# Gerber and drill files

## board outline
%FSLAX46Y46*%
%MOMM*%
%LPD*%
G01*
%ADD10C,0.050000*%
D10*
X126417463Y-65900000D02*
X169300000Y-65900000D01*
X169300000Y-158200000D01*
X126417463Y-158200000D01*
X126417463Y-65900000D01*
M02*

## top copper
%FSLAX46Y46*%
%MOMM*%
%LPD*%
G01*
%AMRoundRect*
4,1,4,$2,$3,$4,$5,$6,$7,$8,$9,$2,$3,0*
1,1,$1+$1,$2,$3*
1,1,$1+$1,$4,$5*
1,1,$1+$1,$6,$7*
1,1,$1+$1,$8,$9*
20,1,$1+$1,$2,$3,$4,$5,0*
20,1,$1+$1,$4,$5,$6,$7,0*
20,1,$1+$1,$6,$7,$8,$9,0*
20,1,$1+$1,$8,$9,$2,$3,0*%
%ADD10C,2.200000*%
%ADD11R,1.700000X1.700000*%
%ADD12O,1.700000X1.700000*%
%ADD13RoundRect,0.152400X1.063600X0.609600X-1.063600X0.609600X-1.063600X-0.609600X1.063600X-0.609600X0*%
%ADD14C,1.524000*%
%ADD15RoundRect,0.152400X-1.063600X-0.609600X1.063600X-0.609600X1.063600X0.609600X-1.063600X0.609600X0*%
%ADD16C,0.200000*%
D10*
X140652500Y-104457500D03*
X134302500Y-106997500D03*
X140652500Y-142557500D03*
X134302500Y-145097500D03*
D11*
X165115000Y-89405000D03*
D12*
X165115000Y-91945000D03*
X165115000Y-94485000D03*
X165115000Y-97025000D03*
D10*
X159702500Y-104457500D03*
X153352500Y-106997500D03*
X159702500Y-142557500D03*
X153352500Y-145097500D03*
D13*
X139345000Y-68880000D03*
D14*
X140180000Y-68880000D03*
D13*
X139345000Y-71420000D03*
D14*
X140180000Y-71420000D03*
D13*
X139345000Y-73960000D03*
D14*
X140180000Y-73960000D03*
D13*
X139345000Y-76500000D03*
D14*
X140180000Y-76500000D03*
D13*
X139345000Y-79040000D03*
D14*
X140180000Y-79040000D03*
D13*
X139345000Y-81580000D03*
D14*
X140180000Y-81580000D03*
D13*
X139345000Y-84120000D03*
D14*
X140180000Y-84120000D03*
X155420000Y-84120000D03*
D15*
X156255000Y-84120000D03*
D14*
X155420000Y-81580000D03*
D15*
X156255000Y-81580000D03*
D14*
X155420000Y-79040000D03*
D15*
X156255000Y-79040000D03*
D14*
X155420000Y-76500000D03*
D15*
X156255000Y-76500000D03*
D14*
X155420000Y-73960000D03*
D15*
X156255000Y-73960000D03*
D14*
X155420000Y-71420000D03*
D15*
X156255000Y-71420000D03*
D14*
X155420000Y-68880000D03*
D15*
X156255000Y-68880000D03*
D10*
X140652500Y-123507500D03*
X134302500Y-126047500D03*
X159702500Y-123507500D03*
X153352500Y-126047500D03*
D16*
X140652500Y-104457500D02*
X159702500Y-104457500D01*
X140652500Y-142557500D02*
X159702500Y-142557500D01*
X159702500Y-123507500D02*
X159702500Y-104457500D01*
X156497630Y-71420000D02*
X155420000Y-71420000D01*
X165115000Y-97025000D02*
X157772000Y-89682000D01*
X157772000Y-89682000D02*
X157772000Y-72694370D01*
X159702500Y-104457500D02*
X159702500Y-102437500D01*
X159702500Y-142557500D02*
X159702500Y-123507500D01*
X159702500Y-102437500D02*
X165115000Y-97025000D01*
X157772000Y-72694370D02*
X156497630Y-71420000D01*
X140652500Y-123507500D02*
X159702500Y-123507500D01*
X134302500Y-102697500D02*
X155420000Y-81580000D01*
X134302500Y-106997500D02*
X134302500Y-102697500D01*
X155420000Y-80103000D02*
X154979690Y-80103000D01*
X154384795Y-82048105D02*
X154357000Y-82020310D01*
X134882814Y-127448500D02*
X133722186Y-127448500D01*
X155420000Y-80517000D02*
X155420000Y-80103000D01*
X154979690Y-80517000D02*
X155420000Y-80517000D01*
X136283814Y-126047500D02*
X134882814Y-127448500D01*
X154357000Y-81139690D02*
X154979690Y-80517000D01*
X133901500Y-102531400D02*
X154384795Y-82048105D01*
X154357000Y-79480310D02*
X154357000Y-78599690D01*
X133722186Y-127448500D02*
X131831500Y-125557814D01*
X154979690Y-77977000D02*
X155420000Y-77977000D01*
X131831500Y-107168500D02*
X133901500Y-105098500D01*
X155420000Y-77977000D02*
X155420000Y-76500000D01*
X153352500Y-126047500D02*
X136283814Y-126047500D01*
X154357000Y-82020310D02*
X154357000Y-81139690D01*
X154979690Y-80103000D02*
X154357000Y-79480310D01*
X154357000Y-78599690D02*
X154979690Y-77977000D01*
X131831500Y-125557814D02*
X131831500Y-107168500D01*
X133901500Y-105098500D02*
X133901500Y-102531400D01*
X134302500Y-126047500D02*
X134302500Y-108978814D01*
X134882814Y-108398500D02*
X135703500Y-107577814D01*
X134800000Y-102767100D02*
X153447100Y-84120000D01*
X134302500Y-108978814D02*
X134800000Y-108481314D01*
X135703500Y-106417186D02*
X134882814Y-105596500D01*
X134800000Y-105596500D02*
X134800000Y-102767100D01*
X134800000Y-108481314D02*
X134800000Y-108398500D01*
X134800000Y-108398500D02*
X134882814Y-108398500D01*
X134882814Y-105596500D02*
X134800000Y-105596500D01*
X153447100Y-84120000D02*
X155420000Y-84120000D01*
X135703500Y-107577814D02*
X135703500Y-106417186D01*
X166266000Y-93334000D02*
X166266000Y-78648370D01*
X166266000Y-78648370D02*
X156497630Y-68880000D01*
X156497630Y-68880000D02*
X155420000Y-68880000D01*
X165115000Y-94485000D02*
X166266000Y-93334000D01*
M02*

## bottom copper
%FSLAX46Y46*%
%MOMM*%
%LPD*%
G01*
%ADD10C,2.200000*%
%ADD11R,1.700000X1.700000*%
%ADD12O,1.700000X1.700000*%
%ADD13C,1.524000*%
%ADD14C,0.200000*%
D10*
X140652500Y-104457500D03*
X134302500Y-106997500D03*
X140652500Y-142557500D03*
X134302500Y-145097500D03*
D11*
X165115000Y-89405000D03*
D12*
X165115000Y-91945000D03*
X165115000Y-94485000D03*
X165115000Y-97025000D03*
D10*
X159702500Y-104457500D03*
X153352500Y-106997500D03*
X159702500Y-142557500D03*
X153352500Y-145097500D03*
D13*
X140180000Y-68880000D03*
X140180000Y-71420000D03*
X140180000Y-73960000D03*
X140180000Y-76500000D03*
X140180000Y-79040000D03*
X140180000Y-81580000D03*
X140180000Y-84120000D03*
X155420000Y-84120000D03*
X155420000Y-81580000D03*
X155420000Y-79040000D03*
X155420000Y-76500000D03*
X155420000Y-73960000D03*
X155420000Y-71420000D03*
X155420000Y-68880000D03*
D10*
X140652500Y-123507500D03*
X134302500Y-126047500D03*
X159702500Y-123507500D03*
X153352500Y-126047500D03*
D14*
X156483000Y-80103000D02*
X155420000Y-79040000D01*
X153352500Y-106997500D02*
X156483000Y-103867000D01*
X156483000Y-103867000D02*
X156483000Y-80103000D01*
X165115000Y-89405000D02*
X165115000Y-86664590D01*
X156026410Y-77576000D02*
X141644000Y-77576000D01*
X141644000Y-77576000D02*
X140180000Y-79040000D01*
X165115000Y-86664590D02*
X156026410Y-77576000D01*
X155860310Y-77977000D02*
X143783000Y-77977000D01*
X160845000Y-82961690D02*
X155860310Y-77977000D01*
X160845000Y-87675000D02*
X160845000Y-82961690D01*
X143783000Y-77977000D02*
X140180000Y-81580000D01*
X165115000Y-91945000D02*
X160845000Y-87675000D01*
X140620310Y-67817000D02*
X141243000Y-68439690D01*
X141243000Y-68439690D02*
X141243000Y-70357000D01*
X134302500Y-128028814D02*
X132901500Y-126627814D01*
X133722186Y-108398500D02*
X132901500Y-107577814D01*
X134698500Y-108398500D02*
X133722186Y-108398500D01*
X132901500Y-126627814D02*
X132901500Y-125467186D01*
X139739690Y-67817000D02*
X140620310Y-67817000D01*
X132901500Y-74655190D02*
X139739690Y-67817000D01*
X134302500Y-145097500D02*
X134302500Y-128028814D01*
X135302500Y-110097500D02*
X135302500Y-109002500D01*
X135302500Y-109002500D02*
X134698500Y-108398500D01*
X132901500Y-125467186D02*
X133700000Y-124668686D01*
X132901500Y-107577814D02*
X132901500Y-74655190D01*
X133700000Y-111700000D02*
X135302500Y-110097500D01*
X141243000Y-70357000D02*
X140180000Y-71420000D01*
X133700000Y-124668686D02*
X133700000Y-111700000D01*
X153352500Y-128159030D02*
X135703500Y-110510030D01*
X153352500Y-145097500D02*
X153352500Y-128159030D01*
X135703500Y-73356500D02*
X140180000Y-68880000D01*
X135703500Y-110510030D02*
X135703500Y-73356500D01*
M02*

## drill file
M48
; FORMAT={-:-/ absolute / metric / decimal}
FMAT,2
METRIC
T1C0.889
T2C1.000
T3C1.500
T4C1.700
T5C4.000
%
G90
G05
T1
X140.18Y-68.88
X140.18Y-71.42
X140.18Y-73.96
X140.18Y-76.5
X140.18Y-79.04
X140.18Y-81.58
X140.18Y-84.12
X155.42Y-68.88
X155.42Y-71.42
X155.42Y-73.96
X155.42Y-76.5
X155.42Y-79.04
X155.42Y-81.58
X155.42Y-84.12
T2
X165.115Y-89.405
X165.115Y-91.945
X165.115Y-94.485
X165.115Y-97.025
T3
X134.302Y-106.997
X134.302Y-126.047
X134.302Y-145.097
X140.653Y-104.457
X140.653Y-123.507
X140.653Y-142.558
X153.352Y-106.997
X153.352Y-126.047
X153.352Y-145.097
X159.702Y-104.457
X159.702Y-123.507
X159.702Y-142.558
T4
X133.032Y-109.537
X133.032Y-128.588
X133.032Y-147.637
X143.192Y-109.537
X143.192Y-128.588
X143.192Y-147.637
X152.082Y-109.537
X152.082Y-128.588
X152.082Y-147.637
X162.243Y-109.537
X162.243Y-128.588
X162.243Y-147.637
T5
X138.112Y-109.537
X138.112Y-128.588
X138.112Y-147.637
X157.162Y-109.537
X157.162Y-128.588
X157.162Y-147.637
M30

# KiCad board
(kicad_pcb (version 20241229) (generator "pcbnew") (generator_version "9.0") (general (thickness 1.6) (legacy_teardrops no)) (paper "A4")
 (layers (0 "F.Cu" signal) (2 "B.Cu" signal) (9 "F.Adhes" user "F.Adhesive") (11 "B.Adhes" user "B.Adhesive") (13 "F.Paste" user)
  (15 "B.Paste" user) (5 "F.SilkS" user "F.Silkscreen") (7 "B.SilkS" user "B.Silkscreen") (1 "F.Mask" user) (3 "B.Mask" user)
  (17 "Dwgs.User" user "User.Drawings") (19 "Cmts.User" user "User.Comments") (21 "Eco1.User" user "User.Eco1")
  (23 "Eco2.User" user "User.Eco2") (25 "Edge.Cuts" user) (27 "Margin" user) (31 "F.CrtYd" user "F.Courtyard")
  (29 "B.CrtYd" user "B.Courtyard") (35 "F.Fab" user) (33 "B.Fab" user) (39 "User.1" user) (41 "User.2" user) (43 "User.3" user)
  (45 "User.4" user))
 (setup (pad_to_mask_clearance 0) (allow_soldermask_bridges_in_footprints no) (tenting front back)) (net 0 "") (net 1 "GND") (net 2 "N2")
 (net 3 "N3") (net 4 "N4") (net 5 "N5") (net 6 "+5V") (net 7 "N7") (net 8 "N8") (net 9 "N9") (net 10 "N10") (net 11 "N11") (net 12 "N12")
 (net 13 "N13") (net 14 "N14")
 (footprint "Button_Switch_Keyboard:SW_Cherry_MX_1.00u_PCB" (layer "F.Cu") (at 140.6525 104.4575)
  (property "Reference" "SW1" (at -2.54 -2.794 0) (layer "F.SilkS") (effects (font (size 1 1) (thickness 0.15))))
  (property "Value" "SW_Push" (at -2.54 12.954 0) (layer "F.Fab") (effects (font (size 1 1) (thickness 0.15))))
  (pad "" np_thru_hole circle (at -7.62 5.08) (size 1.7 1.7) (drill 1.7) (layers "*.Cu" "*.Mask"))
  (pad "" np_thru_hole circle (at -2.54 5.08) (size 4 4) (drill 4) (layers "*.Cu" "*.Mask"))
  (pad "" np_thru_hole circle (at 2.54 5.08) (size 1.7 1.7) (drill 1.7) (layers "*.Cu" "*.Mask"))
  (pad "1" thru_hole circle (at 0 0) (size 2.2 2.2) (drill 1.5) (layers "*.Cu" "*.Mask") (remove_unused_layers no) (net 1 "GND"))
  (pad "2" thru_hole circle (at -6.35 2.54) (size 2.2 2.2) (drill 1.5) (layers "*.Cu" "*.Mask") (remove_unused_layers no) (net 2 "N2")))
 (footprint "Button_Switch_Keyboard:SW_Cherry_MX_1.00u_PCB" (layer "F.Cu") (at 140.6525 142.5575)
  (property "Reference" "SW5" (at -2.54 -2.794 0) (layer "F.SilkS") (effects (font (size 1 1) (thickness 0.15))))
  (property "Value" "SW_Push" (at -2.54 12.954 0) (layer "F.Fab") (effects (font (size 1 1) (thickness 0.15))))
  (pad "" np_thru_hole circle (at -7.62 5.08) (size 1.7 1.7) (drill 1.7) (layers "*.Cu" "*.Mask"))
  (pad "" np_thru_hole circle (at -2.54 5.08) (size 4 4) (drill 4) (layers "*.Cu" "*.Mask"))
  (pad "" np_thru_hole circle (at 2.54 5.08) (size 1.7 1.7) (drill 1.7) (layers "*.Cu" "*.Mask"))
  (pad "1" thru_hole circle (at 0 0) (size 2.2 2.2) (drill 1.5) (layers "*.Cu" "*.Mask") (remove_unused_layers no) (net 1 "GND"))
  (pad "2" thru_hole circle (at -6.35 2.54) (size 2.2 2.2) (drill 1.5) (layers "*.Cu" "*.Mask") (remove_unused_layers no) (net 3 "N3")))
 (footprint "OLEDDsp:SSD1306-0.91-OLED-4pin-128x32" (layer "F.Cu") (at 128.615 87.215)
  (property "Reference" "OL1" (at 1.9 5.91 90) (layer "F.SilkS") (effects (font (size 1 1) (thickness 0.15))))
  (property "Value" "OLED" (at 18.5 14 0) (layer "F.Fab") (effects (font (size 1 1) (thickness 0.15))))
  (pad "1" thru_hole rect (at 36.5 2.19) (size 1.7 1.7) (drill 1) (layers "*.Cu" "*.Mask") (remove_unused_layers no) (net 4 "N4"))
  (pad "2" thru_hole oval (at 36.5 4.73) (size 1.7 1.7) (drill 1) (layers "*.Cu" "*.Mask") (remove_unused_layers no) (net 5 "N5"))
  (pad "3" thru_hole oval (at 36.5 7.27) (size 1.7 1.7) (drill 1) (layers "*.Cu" "*.Mask") (remove_unused_layers no) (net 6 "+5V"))
  (pad "4" thru_hole oval (at 36.5 9.81) (size 1.7 1.7) (drill 1) (layers "*.Cu" "*.Mask") (remove_unused_layers no) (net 1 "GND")))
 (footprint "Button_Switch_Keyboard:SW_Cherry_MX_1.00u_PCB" (layer "F.Cu") (at 159.7025 104.4575)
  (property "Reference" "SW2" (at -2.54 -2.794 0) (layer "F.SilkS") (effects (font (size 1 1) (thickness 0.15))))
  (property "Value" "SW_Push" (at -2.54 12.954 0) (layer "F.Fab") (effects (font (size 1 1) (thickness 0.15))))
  (pad "" np_thru_hole circle (at -7.62 5.08) (size 1.7 1.7) (drill 1.7) (layers "*.Cu" "*.Mask"))
  (pad "" np_thru_hole circle (at -2.54 5.08) (size 4 4) (drill 4) (layers "*.Cu" "*.Mask"))
  (pad "" np_thru_hole circle (at 2.54 5.08) (size 1.7 1.7) (drill 1.7) (layers "*.Cu" "*.Mask"))
  (pad "1" thru_hole circle (at 0 0) (size 2.2 2.2) (drill 1.5) (layers "*.Cu" "*.Mask") (remove_unused_layers no) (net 1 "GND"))
  (pad "2" thru_hole circle (at -6.35 2.54) (size 2.2 2.2) (drill 1.5) (layers "*.Cu" "*.Mask") (remove_unused_layers no) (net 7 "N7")))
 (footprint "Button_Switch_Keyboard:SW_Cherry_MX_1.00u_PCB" (layer "F.Cu") (at 159.7025 142.5575)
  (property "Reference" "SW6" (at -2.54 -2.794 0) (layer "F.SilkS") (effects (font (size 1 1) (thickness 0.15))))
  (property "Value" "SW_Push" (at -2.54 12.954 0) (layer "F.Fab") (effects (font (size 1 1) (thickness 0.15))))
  (pad "" np_thru_hole circle (at -7.62 5.08) (size 1.7 1.7) (drill 1.7) (layers "*.Cu" "*.Mask"))
  (pad "" np_thru_hole circle (at -2.54 5.08) (size 4 4) (drill 4) (layers "*.Cu" "*.Mask"))
  (pad "" np_thru_hole circle (at 2.54 5.08) (size 1.7 1.7) (drill 1.7) (layers "*.Cu" "*.Mask"))
  (pad "1" thru_hole circle (at 0 0) (size 2.2 2.2) (drill 1.5) (layers "*.Cu" "*.Mask") (remove_unused_layers no) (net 1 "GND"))
  (pad "2" thru_hole circle (at -6.35 2.54) (size 2.2 2.2) (drill 1.5) (layers "*.Cu" "*.Mask") (remove_unused_layers no) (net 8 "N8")))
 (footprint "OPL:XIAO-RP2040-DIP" (layer "F.Cu") (at 147.8 76.5)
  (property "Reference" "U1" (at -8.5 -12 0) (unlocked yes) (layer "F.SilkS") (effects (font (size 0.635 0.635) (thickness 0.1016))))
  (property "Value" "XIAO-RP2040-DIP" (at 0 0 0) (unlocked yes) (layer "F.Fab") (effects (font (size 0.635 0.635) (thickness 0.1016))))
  (pad "1" smd roundrect (at -8.455 -7.62 180) (size 2.432 1.524) (layers "F.Cu" "F.Mask") (roundrect_rratio 0.1) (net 8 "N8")
   (thermal_bridge_angle 45))
  (pad "1" thru_hole circle (at -7.62 -7.62 180) (size 1.524 1.524) (drill 0.889) (layers "*.Cu" "*.Mask") (remove_unused_layers no)
   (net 8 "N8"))
  (pad "2" smd roundrect (at -8.455 -5.08 180) (size 2.432 1.524) (layers "F.Cu" "F.Mask") (roundrect_rratio 0.1) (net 3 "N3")
   (thermal_bridge_angle 45))
  (pad "2" thru_hole circle (at -7.62 -5.08 180) (size 1.524 1.524) (drill 0.889) (layers "*.Cu" "*.Mask") (remove_unused_layers no)
   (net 3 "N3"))
  (pad "3" smd roundrect (at -8.455 -2.54 180) (size 2.432 1.524) (layers "F.Cu" "F.Mask") (roundrect_rratio 0.1) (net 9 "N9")
   (thermal_bridge_angle 45))
  (pad "3" thru_hole circle (at -7.62 -2.54 180) (size 1.524 1.524) (drill 0.889) (layers "*.Cu" "*.Mask") (remove_unused_layers no)
   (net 9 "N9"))
  (pad "4" smd roundrect (at -8.455 0 180) (size 2.432 1.524) (layers "F.Cu" "F.Mask") (roundrect_rratio 0.1) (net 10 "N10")
   (thermal_bridge_angle 45))
  (pad "4" thru_hole circle (at -7.62 0 180) (size 1.524 1.524) (drill 0.889) (layers "*.Cu" "*.Mask") (remove_unused_layers no)
   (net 10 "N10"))
  (pad "5" smd roundrect (at -8.455 2.54 180) (size 2.432 1.524) (layers "F.Cu" "F.Mask") (roundrect_rratio 0.1) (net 4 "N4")
   (thermal_bridge_angle 45))
  (pad "5" thru_hole circle (at -7.62 2.54 180) (size 1.524 1.524) (drill 0.889) (layers "*.Cu" "*.Mask") (remove_unused_layers no)
   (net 4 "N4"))
  (pad "6" smd roundrect (at -8.455 5.08 180) (size 2.432 1.524) (layers "F.Cu" "F.Mask") (roundrect_rratio 0.1) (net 5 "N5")
   (thermal_bridge_angle 45))
  (pad "6" thru_hole circle (at -7.62 5.08 180) (size 1.524 1.524) (drill 0.889) (layers "*.Cu" "*.Mask") (remove_unused_layers no)
   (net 5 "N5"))
  (pad "7" smd roundrect (at -8.455 7.62 180) (size 2.432 1.524) (layers "F.Cu" "F.Mask") (roundrect_rratio 0.1) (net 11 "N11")
   (thermal_bridge_angle 45))
  (pad "7" thru_hole circle (at -7.62 7.62 180) (size 1.524 1.524) (drill 0.889) (layers "*.Cu" "*.Mask") (remove_unused_layers no)
   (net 11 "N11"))
  (pad "8" thru_hole circle (at 7.62 7.62) (size 1.524 1.524) (drill 0.889) (layers "*.Cu" "*.Mask") (remove_unused_layers no)
   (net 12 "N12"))
  (pad "8" smd roundrect (at 8.455 7.62) (size 2.432 1.524) (layers "F.Cu" "F.Mask") (roundrect_rratio 0.1) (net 12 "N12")
   (thermal_bridge_angle 45))
  (pad "9" thru_hole circle (at 7.62 5.08) (size 1.524 1.524) (drill 0.889) (layers "*.Cu" "*.Mask") (remove_unused_layers no) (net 2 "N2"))
  (pad "9" smd roundrect (at 8.455 5.08) (size 2.432 1.524) (layers "F.Cu" "F.Mask") (roundrect_rratio 0.1) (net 2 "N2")
   (thermal_bridge_angle 45))
  (pad "10" thru_hole circle (at 7.62 2.54) (size 1.524 1.524) (drill 0.889) (layers "*.Cu" "*.Mask") (remove_unused_layers no) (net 7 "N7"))
  (pad "10" smd roundrect (at 8.455 2.54) (size 2.432 1.524) (layers "F.Cu" "F.Mask") (roundrect_rratio 0.1) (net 7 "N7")
   (thermal_bridge_angle 45))
  (pad "11" thru_hole circle (at 7.62 0) (size 1.524 1.524) (drill 0.889) (layers "*.Cu" "*.Mask") (remove_unused_layers no) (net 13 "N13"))
  (pad "11" smd roundrect (at 8.455 0) (size 2.432 1.524) (layers "F.Cu" "F.Mask") (roundrect_rratio 0.1) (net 13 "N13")
   (thermal_bridge_angle 45))
  (pad "12" thru_hole circle (at 7.62 -2.54) (size 1.524 1.524) (drill 0.889) (layers "*.Cu" "*.Mask") (remove_unused_layers no)
   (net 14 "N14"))
  (pad "12" smd roundrect (at 8.455 -2.54) (size 2.432 1.524) (layers "F.Cu" "F.Mask") (roundrect_rratio 0.1) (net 14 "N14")
   (thermal_bridge_angle 45))
  (pad "13" thru_hole circle (at 7.62 -5.08) (size 1.524 1.524) (drill 0.889) (layers "*.Cu" "*.Mask") (remove_unused_layers no)
   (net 1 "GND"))
  (pad "13" smd roundrect (at 8.455 -5.08) (size 2.432 1.524) (layers "F.Cu" "F.Mask") (roundrect_rratio 0.1) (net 1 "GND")
   (thermal_bridge_angle 45))
  (pad "14" thru_hole circle (at 7.62 -7.62) (size 1.524 1.524) (drill 0.889) (layers "*.Cu" "*.Mask") (remove_unused_layers no)
   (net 6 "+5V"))
  (pad "14" smd roundrect (at 8.455 -7.62) (size 2.432 1.524) (layers "F.Cu" "F.Mask") (roundrect_rratio 0.1) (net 6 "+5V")
   (thermal_bridge_angle 45)))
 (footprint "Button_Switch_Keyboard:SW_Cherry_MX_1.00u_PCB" (layer "F.Cu") (at 140.6525 123.5075)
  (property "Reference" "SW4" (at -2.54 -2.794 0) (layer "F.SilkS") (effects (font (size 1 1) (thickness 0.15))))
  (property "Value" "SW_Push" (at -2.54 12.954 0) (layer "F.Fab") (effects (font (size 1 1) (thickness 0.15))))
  (pad "" np_thru_hole circle (at -7.62 5.08) (size 1.7 1.7) (drill 1.7) (layers "*.Cu" "*.Mask"))
  (pad "" np_thru_hole circle (at -2.54 5.08) (size 4 4) (drill 4) (layers "*.Cu" "*.Mask"))
  (pad "" np_thru_hole circle (at 2.54 5.08) (size 1.7 1.7) (drill 1.7) (layers "*.Cu" "*.Mask"))
  (pad "1" thru_hole circle (at 0 0) (size 2.2 2.2) (drill 1.5) (layers "*.Cu" "*.Mask") (remove_unused_layers no) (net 1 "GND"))
  (pad "2" thru_hole circle (at -6.35 2.54) (size 2.2 2.2) (drill 1.5) (layers "*.Cu" "*.Mask") (remove_unused_layers no) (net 12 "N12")))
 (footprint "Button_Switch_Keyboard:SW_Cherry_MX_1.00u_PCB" (layer "F.Cu") (at 159.7025 123.5075)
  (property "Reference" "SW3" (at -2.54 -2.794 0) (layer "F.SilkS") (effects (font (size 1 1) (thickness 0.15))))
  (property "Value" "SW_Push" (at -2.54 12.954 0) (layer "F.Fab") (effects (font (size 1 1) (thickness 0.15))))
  (pad "" np_thru_hole circle (at -7.62 5.08) (size 1.7 1.7) (drill 1.7) (layers "*.Cu" "*.Mask"))
  (pad "" np_thru_hole circle (at -2.54 5.08) (size 4 4) (drill 4) (layers "*.Cu" "*.Mask"))
  (pad "" np_thru_hole circle (at 2.54 5.08) (size 1.7 1.7) (drill 1.7) (layers "*.Cu" "*.Mask"))
  (pad "1" thru_hole circle (at 0 0) (size 2.2 2.2) (drill 1.5) (layers "*.Cu" "*.Mask") (remove_unused_layers no) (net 1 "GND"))
  (pad "2" thru_hole circle (at -6.35 2.54) (size 2.2 2.2) (drill 1.5) (layers "*.Cu" "*.Mask") (remove_unused_layers no) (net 13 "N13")))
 (gr_rect (start 126.417463 65.9) (end 169.3 158.2) (stroke (width 0.05) (type default)) (fill no) (layer "Edge.Cuts"))
 (segment (start 140.6525 104.4575) (end 159.7025 104.4575) (width 0.2) (layer "F.Cu") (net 1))
 (segment (start 140.6525 142.5575) (end 159.7025 142.5575) (width 0.2) (layer "F.Cu") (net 1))
 (segment (start 159.7025 123.5075) (end 159.7025 104.4575) (width 0.2) (layer "F.Cu") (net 1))
 (segment (start 156.49763 71.42) (end 155.42 71.42) (width 0.2) (layer "F.Cu") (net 1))
 (segment (start 165.115 97.025) (end 157.772 89.682) (width 0.2) (layer "F.Cu") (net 1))
 (segment (start 157.772 89.682) (end 157.772 72.69437) (width 0.2) (layer "F.Cu") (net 1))
 (segment (start 159.7025 104.4575) (end 159.7025 102.4375) (width 0.2) (layer "F.Cu") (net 1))
 (segment (start 159.7025 142.5575) (end 159.7025 123.5075) (width 0.2) (layer "F.Cu") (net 1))
 (segment (start 159.7025 102.4375) (end 165.115 97.025) (width 0.2) (layer "F.Cu") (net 1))
 (segment (start 157.772 72.69437) (end 156.49763 71.42) (width 0.2) (layer "F.Cu") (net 1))
 (segment (start 140.6525 123.5075) (end 159.7025 123.5075) (width 0.2) (layer "F.Cu") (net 1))
 (segment (start 134.3025 102.6975) (end 155.42 81.58) (width 0.2) (layer "F.Cu") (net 2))
 (segment (start 134.3025 106.9975) (end 134.3025 102.6975) (width 0.2) (layer "F.Cu") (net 2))
 (segment (start 156.483 80.103) (end 155.42 79.04) (width 0.2) (layer "B.Cu") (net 7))
 (segment (start 153.3525 106.9975) (end 156.483 103.867) (width 0.2) (layer "B.Cu") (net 7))
 (segment (start 156.483 103.867) (end 156.483 80.103) (width 0.2) (layer "B.Cu") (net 7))
 (segment (start 155.42 80.103) (end 154.97969 80.103) (width 0.2) (layer "F.Cu") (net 13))
 (segment (start 154.384795 82.048105) (end 154.357 82.02031) (width 0.2) (layer "F.Cu") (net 13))
 (segment (start 134.882814 127.4485) (end 133.722186 127.4485) (width 0.2) (layer "F.Cu") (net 13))
 (segment (start 155.42 80.517) (end 155.42 80.103) (width 0.2) (layer "F.Cu") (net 13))
 (segment (start 154.97969 80.517) (end 155.42 80.517) (width 0.2) (layer "F.Cu") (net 13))
 (segment (start 136.283814 126.0475) (end 134.882814 127.4485) (width 0.2) (layer "F.Cu") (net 13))
 (segment (start 154.357 81.13969) (end 154.97969 80.517) (width 0.2) (layer "F.Cu") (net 13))
 (segment (start 133.9015 102.5314) (end 154.384795 82.048105) (width 0.2) (layer "F.Cu") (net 13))
 (segment (start 154.357 79.48031) (end 154.357 78.59969) (width 0.2) (layer "F.Cu") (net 13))
 (segment (start 133.722186 127.4485) (end 131.8315 125.557814) (width 0.2) (layer "F.Cu") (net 13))
 (segment (start 154.97969 77.977) (end 155.42 77.977) (width 0.2) (layer "F.Cu") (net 13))
 (segment (start 131.8315 107.1685) (end 133.9015 105.0985) (width 0.2) (layer "F.Cu") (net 13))
 (segment (start 155.42 77.977) (end 155.42 76.5) (width 0.2) (layer "F.Cu") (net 13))
 (segment (start 153.3525 126.0475) (end 136.283814 126.0475) (width 0.2) (layer "F.Cu") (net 13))
 (segment (start 154.357 82.02031) (end 154.357 81.13969) (width 0.2) (layer "F.Cu") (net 13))
 (segment (start 154.97969 80.103) (end 154.357 79.48031) (width 0.2) (layer "F.Cu") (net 13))
 (segment (start 154.357 78.59969) (end 154.97969 77.977) (width 0.2) (layer "F.Cu") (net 13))
 (segment (start 131.8315 125.557814) (end 131.8315 107.1685) (width 0.2) (layer "F.Cu") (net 13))
 (segment (start 133.9015 105.0985) (end 133.9015 102.5314) (width 0.2) (layer "F.Cu") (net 13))
 (segment (start 134.3025 126.0475) (end 134.3025 108.978814) (width 0.2) (layer "F.Cu") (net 12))
 (segment (start 134.882814 108.3985) (end 135.7035 107.577814) (width 0.2) (layer "F.Cu") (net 12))
 (segment (start 134.8 102.7671) (end 153.4471 84.12) (width 0.2) (layer "F.Cu") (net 12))
 (segment (start 134.3025 108.978814) (end 134.8 108.481314) (width 0.2) (layer "F.Cu") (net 12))
 (segment (start 135.7035 106.417186) (end 134.882814 105.5965) (width 0.2) (layer "F.Cu") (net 12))
 (segment (start 134.8 105.5965) (end 134.8 102.7671) (width 0.2) (layer "F.Cu") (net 12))
 (segment (start 134.8 108.481314) (end 134.8 108.3985) (width 0.2) (layer "F.Cu") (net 12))
 (segment (start 134.8 108.3985) (end 134.882814 108.3985) (width 0.2) (layer "F.Cu") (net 12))
 (segment (start 134.882814 105.5965) (end 134.8 105.5965) (width 0.2) (layer "F.Cu") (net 12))
 (segment (start 153.4471 84.12) (end 155.42 84.12) (width 0.2) (layer "F.Cu") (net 12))
 (segment (start 135.7035 107.577814) (end 135.7035 106.417186) (width 0.2) (layer "F.Cu") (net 12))
 (segment (start 165.115 89.405) (end 165.115 86.66459) (width 0.2) (layer "B.Cu") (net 4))
 (segment (start 156.02641 77.576) (end 141.644 77.576) (width 0.2) (layer "B.Cu") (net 4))
 (segment (start 141.644 77.576) (end 140.18 79.04) (width 0.2) (layer "B.Cu") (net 4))
 (segment (start 165.115 86.66459) (end 156.02641 77.576) (width 0.2) (layer "B.Cu") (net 4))
 (segment (start 155.86031 77.977) (end 143.783 77.977) (width 0.2) (layer "B.Cu") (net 5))
 (segment (start 160.845 82.96169) (end 155.86031 77.977) (width 0.2) (layer "B.Cu") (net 5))
 (segment (start 160.845 87.675) (end 160.845 82.96169) (width 0.2) (layer "B.Cu") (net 5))
 (segment (start 143.783 77.977) (end 140.18 81.58) (width 0.2) (layer "B.Cu") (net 5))
 (segment (start 165.115 91.945) (end 160.845 87.675) (width 0.2) (layer "B.Cu") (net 5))
 (segment (start 166.266 93.334) (end 166.266 78.64837) (width 0.2) (layer "F.Cu") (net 6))
 (segment (start 166.266 78.64837) (end 156.49763 68.88) (width 0.2) (layer "F.Cu") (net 6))
 (segment (start 156.49763 68.88) (end 155.42 68.88) (width 0.2) (layer "F.Cu") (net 6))
 (segment (start 165.115 94.485) (end 166.266 93.334) (width 0.2) (layer "F.Cu") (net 6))
 (segment (start 140.62031 67.817) (end 141.243 68.43969) (width 0.2) (layer "B.Cu") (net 3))
 (segment (start 141.243 68.43969) (end 141.243 70.357) (width 0.2) (layer "B.Cu") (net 3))
 (segment (start 134.3025 128.028814) (end 132.9015 126.627814) (width 0.2) (layer "B.Cu") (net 3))
 (segment (start 133.722186 108.3985) (end 132.9015 107.577814) (width 0.2) (layer "B.Cu") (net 3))
 (segment (start 134.6985 108.3985) (end 133.722186 108.3985) (width 0.2) (layer "B.Cu") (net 3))
 (segment (start 132.9015 126.627814) (end 132.9015 125.467186) (width 0.2) (layer "B.Cu") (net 3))
 (segment (start 139.73969 67.817) (end 140.62031 67.817) (width 0.2) (layer "B.Cu") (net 3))
 (segment (start 132.9015 74.65519) (end 139.73969 67.817) (width 0.2) (layer "B.Cu") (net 3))
 (segment (start 134.3025 145.0975) (end 134.3025 128.028814) (width 0.2) (layer "B.Cu") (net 3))
 (segment (start 135.3025 110.0975) (end 135.3025 109.0025) (width 0.2) (layer "B.Cu") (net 3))
 (segment (start 135.3025 109.0025) (end 134.6985 108.3985) (width 0.2) (layer "B.Cu") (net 3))
 (segment (start 132.9015 125.467186) (end 133.7 124.668686) (width 0.2) (layer "B.Cu") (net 3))
 (segment (start 132.9015 107.577814) (end 132.9015 74.65519) (width 0.2) (layer "B.Cu") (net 3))
 (segment (start 133.7 111.7) (end 135.3025 110.0975) (width 0.2) (layer "B.Cu") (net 3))
 (segment (start 141.243 70.357) (end 140.18 71.42) (width 0.2) (layer "B.Cu") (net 3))
 (segment (start 133.7 124.668686) (end 133.7 111.7) (width 0.2) (layer "B.Cu") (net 3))
 (segment (start 153.3525 128.15903) (end 135.7035 110.51003) (width 0.2) (layer "B.Cu") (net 8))
 (segment (start 153.3525 145.0975) (end 153.3525 128.15903) (width 0.2) (layer "B.Cu") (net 8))
 (segment (start 135.7035 73.3565) (end 140.18 68.88) (width 0.2) (layer "B.Cu") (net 8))
 (segment (start 135.7035 110.51003) (end 135.7035 73.3565) (width 0.2) (layer "B.Cu") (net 8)))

